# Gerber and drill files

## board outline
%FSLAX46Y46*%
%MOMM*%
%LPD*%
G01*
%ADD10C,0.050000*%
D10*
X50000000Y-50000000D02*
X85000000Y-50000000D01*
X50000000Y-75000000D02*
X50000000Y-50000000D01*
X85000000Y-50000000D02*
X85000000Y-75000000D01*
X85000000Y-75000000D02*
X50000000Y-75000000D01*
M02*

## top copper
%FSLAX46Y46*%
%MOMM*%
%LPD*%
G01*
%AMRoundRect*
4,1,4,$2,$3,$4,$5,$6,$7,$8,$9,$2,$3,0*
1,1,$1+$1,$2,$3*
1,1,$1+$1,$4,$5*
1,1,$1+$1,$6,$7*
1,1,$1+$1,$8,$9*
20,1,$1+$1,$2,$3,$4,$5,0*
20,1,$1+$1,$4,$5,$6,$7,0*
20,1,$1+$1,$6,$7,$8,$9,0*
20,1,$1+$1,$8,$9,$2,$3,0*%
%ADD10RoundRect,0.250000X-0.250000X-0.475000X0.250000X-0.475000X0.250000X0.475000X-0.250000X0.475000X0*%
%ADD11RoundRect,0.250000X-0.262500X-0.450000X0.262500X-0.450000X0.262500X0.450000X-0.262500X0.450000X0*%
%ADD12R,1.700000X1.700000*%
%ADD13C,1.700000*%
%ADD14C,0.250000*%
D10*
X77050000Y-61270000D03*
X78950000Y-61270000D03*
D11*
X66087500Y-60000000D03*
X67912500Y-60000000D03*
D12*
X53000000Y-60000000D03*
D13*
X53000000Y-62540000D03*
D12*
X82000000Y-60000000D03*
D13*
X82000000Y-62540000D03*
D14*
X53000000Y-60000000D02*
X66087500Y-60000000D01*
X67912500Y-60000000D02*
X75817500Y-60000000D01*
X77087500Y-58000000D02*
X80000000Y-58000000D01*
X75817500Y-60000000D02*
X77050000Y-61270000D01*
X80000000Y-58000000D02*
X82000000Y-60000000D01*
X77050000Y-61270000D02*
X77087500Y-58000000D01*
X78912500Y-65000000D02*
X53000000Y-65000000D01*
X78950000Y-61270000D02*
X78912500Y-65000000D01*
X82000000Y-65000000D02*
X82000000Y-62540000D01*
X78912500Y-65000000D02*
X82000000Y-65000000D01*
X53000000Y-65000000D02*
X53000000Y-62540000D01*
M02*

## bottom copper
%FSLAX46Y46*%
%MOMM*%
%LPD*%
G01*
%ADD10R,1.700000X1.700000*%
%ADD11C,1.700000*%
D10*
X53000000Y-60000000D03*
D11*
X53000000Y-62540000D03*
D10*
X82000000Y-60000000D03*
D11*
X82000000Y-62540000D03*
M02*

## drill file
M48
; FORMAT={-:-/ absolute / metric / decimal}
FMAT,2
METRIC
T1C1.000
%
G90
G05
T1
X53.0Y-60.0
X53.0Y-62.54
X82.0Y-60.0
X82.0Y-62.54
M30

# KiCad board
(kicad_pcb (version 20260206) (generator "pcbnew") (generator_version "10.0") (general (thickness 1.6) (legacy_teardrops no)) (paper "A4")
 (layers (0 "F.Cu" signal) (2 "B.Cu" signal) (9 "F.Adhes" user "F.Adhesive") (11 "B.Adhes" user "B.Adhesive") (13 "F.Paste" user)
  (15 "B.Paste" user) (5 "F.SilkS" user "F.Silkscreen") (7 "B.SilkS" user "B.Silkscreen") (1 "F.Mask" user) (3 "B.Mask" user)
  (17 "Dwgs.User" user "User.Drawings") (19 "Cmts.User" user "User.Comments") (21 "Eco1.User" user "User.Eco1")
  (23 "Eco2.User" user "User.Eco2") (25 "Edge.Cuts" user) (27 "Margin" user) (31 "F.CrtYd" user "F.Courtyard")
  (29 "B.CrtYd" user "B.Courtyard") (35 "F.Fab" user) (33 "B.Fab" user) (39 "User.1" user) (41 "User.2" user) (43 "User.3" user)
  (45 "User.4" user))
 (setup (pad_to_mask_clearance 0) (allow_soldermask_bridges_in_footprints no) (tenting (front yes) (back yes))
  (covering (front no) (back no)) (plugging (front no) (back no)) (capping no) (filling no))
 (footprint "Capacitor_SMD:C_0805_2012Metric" (layer "F.Cu") (at 78 61.27)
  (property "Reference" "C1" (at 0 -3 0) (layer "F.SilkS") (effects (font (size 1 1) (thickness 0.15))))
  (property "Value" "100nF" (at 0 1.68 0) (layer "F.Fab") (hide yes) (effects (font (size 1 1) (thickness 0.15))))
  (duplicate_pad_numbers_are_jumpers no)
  (pad "1" smd roundrect (at -0.95 0) (size 1 1.45) (layers "F.Cu" "F.Mask" "F.Paste") (roundrect_rratio 0.25) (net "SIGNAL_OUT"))
  (pad "2" smd roundrect (at 0.95 0) (size 1 1.45) (layers "F.Cu" "F.Mask" "F.Paste") (roundrect_rratio 0.25) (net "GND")))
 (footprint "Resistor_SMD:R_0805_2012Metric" (layer "F.Cu") (at 67 60)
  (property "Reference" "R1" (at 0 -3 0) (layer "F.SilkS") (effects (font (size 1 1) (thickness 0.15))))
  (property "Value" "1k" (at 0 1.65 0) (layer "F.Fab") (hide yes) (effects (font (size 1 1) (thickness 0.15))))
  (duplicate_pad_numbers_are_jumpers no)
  (pad "1" smd roundrect (at -0.9125 0) (size 1.025 1.4) (layers "F.Cu" "F.Mask" "F.Paste") (roundrect_rratio 0.243902) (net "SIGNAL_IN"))
  (pad "2" smd roundrect (at 0.9125 0) (size 1.025 1.4) (layers "F.Cu" "F.Mask" "F.Paste") (roundrect_rratio 0.243902) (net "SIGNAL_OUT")))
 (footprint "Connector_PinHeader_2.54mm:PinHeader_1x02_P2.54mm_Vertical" (layer "F.Cu") (at 53 60)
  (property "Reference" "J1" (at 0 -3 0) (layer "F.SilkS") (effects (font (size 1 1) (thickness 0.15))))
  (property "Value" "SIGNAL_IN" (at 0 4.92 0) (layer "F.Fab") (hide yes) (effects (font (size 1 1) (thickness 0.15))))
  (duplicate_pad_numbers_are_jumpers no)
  (pad "1" thru_hole rect (at 0 0) (size 1.7 1.7) (drill 1) (layers "*.Cu" "*.Mask") (remove_unused_layers no) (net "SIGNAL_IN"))
  (pad "2" thru_hole circle (at 0 2.54) (size 1.7 1.7) (drill 1) (layers "*.Cu" "*.Mask") (remove_unused_layers no) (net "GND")))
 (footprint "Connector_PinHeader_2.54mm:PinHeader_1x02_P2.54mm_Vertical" (layer "F.Cu") (at 82 60)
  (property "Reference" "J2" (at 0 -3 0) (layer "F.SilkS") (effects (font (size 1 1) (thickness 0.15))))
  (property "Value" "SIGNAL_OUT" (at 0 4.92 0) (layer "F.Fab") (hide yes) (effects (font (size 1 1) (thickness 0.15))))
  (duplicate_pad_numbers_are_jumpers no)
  (pad "1" thru_hole rect (at 0 0) (size 1.7 1.7) (drill 1) (layers "*.Cu" "*.Mask") (remove_unused_layers no) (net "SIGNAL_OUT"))
  (pad "2" thru_hole circle (at 0 2.54) (size 1.7 1.7) (drill 1) (layers "*.Cu" "*.Mask") (remove_unused_layers no) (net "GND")))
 (gr_line (start 50 50) (end 85 50) (stroke (width 0.05) (type default)) (layer "Edge.Cuts"))
 (gr_line (start 50 75) (end 50 50) (stroke (width 0.05) (type default)) (layer "Edge.Cuts"))
 (gr_line (start 85 50) (end 85 75) (stroke (width 0.05) (type default)) (layer "Edge.Cuts"))
 (gr_line (start 85 75) (end 50 75) (stroke (width 0.05) (type default)) (layer "Edge.Cuts"))
 (segment (start 53 60) (end 66.0875 60) (width 0.25) (layer "F.Cu") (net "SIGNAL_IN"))
 (segment (start 67.9125 60) (end 75.8175 60) (width 0.25) (layer "F.Cu") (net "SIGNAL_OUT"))
 (segment (start 77.0875 58) (end 80 58) (width 0.25) (layer "F.Cu") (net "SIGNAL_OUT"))
 (segment (start 75.8175 60) (end 77.05 61.27) (width 0.25) (layer "F.Cu") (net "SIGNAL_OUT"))
 (segment (start 80 58) (end 82 60) (width 0.25) (layer "F.Cu") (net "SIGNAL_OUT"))
 (segment (start 77.05 61.27) (end 77.0875 58) (width 0.25) (layer "F.Cu") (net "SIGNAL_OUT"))
 (segment (start 78.9125 65) (end 53 65) (width 0.25) (layer "F.Cu") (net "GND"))
 (segment (start 78.95 61.27) (end 78.9125 65) (width 0.25) (layer "F.Cu") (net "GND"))
 (segment (start 82 65) (end 82 62.54) (width 0.25) (layer "F.Cu") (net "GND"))
 (segment (start 78.9125 65) (end 82 65) (width 0.25) (layer "F.Cu") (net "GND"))
 (segment (start 53 65) (end 53 62.54) (width 0.25) (layer "F.Cu") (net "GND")))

